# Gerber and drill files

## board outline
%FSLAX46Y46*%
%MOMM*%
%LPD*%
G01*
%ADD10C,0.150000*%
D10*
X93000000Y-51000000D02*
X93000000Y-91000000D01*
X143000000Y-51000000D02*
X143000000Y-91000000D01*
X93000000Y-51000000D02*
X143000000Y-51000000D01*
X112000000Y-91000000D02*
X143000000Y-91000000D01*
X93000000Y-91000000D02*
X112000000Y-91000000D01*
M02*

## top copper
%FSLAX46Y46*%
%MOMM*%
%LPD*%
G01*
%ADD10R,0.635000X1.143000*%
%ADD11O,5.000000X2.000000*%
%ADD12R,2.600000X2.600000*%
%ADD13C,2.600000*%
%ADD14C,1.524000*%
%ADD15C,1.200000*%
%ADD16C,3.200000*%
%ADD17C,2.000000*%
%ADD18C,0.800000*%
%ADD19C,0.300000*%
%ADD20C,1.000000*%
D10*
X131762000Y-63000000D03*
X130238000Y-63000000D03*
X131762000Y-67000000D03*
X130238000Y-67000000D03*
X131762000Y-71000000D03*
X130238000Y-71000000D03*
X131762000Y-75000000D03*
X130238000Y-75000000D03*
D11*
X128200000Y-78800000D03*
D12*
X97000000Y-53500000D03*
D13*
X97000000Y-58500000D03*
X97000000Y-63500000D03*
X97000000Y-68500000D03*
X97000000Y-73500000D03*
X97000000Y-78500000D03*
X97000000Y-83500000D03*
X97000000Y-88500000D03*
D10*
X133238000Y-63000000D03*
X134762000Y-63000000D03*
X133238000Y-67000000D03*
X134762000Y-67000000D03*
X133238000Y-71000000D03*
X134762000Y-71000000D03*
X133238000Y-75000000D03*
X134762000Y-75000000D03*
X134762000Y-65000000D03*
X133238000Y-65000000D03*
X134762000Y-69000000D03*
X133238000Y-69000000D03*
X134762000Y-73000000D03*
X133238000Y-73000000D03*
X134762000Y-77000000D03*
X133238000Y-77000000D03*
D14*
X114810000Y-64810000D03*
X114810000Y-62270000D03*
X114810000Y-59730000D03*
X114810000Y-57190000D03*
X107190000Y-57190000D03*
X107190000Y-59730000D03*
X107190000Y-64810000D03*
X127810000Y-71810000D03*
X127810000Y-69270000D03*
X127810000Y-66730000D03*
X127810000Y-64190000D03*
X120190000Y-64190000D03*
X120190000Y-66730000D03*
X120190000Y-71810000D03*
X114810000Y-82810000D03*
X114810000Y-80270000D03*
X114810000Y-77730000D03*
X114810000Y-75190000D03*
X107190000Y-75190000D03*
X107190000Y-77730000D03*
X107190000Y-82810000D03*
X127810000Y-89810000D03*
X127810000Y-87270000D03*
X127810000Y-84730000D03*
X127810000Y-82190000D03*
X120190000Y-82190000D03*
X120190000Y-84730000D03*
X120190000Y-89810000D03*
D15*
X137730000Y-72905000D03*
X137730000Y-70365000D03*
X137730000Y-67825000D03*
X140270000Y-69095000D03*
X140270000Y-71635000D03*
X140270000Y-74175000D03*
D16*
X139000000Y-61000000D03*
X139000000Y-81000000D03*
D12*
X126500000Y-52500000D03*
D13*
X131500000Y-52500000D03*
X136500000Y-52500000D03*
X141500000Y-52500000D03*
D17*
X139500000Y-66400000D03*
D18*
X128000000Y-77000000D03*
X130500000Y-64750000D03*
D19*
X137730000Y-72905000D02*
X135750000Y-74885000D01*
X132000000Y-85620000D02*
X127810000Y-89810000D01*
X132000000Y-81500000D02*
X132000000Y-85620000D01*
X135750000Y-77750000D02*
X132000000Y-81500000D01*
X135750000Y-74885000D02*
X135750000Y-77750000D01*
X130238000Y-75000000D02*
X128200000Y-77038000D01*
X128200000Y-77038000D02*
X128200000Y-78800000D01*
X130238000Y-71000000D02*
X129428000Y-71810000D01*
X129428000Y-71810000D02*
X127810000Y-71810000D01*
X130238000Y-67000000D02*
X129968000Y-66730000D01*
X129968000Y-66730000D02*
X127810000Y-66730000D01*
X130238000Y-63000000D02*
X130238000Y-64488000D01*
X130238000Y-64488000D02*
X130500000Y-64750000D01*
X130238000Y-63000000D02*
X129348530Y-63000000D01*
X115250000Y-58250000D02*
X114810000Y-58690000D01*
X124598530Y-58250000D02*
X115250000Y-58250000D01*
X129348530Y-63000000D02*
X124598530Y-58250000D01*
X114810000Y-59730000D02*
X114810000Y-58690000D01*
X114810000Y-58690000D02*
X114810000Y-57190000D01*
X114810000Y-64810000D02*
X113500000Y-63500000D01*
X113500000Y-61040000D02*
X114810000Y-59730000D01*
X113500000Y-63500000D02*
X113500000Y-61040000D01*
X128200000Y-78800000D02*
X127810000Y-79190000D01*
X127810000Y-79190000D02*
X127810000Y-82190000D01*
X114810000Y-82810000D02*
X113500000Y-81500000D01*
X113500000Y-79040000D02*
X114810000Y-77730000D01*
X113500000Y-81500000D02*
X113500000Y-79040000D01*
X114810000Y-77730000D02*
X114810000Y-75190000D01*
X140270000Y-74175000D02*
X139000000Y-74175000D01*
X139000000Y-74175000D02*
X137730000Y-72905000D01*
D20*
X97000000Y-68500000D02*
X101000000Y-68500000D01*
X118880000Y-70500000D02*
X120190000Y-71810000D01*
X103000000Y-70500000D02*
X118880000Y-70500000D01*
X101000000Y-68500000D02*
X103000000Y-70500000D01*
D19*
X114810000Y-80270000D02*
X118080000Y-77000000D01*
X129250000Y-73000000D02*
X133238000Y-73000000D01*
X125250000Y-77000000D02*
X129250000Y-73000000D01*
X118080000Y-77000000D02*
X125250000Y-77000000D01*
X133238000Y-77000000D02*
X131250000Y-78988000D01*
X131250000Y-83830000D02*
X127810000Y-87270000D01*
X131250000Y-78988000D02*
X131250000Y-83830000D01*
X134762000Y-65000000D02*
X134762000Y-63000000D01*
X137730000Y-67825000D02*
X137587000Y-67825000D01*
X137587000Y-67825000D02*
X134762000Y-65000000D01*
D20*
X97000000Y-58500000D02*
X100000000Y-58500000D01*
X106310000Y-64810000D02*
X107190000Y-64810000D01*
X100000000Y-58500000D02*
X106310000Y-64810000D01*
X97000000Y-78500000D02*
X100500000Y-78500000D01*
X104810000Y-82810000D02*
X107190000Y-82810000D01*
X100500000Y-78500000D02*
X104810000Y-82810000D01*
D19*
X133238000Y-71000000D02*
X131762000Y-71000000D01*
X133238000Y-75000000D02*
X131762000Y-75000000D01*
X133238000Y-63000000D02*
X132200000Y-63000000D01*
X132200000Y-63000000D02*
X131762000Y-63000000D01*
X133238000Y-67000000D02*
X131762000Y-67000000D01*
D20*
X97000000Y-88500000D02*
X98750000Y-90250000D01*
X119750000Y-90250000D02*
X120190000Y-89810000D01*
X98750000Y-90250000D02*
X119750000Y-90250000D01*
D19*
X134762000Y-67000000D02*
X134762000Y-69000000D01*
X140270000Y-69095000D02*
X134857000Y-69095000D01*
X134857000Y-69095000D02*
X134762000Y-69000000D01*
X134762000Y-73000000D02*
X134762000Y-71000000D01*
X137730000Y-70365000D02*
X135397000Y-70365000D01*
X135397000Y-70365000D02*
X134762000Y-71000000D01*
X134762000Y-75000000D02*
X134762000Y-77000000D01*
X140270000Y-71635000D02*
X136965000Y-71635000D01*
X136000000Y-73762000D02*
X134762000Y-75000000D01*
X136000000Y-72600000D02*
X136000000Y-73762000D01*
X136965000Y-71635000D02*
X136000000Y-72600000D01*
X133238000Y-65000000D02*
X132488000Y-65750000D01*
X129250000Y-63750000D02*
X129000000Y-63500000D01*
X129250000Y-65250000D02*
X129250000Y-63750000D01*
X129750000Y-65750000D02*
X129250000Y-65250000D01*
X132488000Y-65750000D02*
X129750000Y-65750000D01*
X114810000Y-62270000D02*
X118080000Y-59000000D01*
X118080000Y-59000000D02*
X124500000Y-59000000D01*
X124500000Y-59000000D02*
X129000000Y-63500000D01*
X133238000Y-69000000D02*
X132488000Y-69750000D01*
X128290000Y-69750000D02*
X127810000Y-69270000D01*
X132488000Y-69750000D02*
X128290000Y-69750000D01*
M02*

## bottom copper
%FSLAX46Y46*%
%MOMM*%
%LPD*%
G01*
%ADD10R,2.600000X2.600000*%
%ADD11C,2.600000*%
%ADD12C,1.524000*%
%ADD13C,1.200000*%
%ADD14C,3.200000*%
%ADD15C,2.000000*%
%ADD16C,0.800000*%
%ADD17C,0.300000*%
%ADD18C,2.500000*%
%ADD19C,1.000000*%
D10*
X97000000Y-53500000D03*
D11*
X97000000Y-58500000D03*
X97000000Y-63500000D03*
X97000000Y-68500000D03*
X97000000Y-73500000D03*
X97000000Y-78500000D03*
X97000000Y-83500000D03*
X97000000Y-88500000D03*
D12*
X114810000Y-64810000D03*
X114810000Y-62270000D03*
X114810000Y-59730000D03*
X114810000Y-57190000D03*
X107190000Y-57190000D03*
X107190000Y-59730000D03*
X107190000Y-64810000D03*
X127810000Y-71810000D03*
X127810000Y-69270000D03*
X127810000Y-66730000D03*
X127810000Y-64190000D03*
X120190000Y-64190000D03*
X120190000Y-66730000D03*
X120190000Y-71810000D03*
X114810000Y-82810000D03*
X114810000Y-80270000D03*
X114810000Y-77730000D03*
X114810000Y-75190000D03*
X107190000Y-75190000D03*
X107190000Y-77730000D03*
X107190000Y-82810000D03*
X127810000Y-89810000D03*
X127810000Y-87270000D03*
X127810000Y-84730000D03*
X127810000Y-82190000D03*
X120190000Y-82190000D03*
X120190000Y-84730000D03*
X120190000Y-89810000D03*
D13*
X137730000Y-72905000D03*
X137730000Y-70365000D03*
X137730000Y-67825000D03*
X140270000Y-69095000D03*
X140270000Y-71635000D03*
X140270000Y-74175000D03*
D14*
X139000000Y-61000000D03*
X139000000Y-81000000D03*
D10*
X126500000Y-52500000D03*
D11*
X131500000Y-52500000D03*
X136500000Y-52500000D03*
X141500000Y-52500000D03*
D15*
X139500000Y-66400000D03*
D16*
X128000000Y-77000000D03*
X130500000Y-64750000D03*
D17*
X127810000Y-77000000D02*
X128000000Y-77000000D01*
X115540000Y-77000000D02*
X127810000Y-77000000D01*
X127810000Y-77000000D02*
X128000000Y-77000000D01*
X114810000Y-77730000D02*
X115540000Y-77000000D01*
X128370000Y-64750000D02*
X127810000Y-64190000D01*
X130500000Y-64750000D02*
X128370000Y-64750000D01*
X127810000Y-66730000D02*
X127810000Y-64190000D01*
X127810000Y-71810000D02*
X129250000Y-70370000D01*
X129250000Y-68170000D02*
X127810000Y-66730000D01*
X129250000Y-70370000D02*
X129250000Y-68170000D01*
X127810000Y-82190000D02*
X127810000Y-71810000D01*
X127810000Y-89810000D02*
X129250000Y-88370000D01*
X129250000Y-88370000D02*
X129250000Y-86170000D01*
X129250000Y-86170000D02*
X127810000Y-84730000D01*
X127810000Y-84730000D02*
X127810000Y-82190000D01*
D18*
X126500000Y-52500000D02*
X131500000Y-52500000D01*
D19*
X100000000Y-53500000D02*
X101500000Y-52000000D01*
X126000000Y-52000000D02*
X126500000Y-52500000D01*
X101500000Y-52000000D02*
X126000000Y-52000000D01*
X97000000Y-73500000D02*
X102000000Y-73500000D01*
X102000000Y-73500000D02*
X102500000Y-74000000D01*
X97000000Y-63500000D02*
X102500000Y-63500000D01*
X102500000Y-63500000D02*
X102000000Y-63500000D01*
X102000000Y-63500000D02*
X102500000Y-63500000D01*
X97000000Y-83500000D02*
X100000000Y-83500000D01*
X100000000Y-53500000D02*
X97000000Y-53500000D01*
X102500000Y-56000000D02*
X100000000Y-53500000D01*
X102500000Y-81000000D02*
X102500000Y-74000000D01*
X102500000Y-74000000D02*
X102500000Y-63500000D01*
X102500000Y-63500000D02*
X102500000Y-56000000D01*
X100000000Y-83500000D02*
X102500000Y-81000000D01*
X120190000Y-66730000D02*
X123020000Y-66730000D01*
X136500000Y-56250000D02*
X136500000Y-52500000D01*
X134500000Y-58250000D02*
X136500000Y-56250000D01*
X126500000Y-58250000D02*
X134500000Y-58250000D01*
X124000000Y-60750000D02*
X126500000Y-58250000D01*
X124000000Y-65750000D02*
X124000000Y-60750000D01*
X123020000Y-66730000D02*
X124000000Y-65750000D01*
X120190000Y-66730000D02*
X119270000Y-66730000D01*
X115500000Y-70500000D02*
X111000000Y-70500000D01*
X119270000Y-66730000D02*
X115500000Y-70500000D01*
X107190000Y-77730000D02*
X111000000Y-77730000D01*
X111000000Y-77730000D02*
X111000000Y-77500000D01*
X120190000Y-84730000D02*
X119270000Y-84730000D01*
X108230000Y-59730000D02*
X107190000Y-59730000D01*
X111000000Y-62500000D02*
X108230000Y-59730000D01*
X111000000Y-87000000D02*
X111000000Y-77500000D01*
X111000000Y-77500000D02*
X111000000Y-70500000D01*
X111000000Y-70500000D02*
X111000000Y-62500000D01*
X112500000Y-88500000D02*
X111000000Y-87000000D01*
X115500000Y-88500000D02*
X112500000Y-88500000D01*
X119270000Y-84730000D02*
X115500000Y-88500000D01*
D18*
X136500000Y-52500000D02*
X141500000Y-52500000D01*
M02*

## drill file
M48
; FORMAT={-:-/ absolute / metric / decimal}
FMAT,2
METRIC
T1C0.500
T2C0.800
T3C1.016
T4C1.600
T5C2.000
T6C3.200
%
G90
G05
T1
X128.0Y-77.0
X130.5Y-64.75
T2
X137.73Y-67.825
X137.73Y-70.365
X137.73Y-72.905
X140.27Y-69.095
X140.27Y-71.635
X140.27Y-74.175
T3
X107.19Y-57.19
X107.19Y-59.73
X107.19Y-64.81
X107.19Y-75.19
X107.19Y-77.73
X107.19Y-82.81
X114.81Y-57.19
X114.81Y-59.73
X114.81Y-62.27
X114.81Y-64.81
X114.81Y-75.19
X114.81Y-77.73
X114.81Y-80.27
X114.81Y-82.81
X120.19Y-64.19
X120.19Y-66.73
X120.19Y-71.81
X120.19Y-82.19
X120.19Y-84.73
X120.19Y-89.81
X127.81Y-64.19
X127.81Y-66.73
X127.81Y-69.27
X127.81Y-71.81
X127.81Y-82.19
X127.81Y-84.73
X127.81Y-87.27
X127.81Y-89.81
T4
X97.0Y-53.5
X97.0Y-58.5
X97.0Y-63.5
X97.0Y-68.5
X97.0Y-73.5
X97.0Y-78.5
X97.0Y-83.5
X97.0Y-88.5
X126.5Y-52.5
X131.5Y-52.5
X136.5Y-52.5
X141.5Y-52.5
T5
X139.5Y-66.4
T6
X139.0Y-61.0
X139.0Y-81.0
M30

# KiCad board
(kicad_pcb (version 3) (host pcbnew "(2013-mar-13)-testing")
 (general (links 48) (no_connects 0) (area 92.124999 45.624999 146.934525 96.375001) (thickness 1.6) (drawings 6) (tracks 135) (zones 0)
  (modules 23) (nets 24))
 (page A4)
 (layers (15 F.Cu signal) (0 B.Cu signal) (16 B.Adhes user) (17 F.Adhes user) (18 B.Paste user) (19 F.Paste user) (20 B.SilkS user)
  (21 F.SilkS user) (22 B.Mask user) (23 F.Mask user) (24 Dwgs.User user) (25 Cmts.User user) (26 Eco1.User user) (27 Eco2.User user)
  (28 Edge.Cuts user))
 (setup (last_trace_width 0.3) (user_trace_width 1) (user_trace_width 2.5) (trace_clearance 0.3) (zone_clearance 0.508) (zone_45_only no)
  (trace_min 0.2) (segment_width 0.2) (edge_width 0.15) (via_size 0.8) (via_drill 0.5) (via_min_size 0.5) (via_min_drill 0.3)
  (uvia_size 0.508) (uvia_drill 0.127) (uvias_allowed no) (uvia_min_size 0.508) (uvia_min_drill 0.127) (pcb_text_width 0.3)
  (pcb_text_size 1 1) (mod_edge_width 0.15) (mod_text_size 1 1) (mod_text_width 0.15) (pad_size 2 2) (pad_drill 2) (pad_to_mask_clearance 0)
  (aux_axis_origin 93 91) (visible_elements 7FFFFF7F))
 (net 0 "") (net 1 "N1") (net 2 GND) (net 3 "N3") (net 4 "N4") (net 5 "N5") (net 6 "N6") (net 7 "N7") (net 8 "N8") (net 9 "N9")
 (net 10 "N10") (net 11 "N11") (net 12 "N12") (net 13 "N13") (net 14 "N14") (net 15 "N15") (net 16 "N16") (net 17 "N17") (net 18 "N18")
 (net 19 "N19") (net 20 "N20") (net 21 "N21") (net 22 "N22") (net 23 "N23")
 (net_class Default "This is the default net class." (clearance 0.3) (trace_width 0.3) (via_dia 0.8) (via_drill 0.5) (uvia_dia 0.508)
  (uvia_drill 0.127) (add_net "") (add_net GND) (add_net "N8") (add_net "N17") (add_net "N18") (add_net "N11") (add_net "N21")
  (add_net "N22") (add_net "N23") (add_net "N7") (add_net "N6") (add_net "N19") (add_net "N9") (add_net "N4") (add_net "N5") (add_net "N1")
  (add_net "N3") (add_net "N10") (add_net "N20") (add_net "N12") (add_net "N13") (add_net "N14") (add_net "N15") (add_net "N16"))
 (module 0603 (layer F.Cu) (at 131 63 180)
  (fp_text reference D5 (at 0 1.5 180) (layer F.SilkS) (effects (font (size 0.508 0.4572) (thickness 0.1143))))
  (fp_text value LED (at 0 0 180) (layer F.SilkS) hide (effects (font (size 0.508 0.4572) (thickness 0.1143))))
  (pad 1 smd rect (at -0.762 0 180) (size 0.635 1.143) (layers F.Cu F.Paste F.Mask) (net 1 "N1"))
  (pad 2 smd rect (at 0.762 0 180) (size 0.635 1.143) (layers F.Cu F.Paste F.Mask) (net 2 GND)))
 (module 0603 (layer F.Cu) (at 131 67 180)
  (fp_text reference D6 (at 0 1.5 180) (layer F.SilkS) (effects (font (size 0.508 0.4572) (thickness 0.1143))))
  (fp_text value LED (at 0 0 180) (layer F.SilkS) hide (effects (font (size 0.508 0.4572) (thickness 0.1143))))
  (pad 1 smd rect (at -0.762 0 180) (size 0.635 1.143) (layers F.Cu F.Paste F.Mask) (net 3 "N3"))
  (pad 2 smd rect (at 0.762 0 180) (size 0.635 1.143) (layers F.Cu F.Paste F.Mask) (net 2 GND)))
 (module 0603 (layer F.Cu) (at 131 71 180)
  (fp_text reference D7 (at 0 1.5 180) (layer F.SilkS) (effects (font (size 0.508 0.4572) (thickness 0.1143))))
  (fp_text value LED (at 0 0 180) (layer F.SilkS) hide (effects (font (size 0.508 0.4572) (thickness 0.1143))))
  (pad 1 smd rect (at -0.762 0 180) (size 0.635 1.143) (layers F.Cu F.Paste F.Mask) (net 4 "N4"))
  (pad 2 smd rect (at 0.762 0 180) (size 0.635 1.143) (layers F.Cu F.Paste F.Mask) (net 2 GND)))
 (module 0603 (layer F.Cu) (at 131 75 180)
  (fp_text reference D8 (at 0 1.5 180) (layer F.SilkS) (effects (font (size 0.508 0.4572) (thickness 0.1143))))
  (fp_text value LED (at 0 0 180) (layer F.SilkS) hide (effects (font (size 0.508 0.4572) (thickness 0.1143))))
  (pad 1 smd rect (at -0.762 0 180) (size 0.635 1.143) (layers F.Cu F.Paste F.Mask) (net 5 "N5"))
  (pad 2 smd rect (at 0.762 0 180) (size 0.635 1.143) (layers F.Cu F.Paste F.Mask) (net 2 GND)))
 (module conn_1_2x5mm (layer F.Cu) (at 128.2 78.8)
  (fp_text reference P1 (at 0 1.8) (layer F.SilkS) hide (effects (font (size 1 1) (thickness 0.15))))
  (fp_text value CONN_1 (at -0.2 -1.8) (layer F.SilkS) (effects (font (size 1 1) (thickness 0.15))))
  (pad 1 smd oval (at 0 0) (size 5 2) (layers F.Cu F.Mask) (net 2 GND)))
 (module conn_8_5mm (layer F.Cu) (at 97 71 270)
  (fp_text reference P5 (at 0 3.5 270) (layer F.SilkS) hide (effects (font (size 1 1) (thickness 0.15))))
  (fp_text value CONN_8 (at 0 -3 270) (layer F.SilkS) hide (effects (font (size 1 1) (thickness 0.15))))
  (pad 1 thru_hole rect (at -17.5 0 270) (size 2.6 2.6) (drill 1.6) (layers *.Cu *.Mask F.SilkS) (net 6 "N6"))
  (pad 2 thru_hole circle (at -12.5 0 270) (size 2.6 2.6) (drill 1.6) (layers *.Cu *.Mask F.SilkS) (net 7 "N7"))
  (pad 3 thru_hole circle (at -7.5 0 270) (size 2.6 2.6) (drill 1.6) (layers *.Cu *.Mask F.SilkS) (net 6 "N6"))
  (pad 4 thru_hole circle (at -2.5 0 270) (size 2.6 2.6) (drill 1.6) (layers *.Cu *.Mask F.SilkS) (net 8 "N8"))
  (pad 5 thru_hole circle (at 2.5 0 270) (size 2.6 2.6) (drill 1.6) (layers *.Cu *.Mask F.SilkS) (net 6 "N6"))
  (pad 6 thru_hole circle (at 7.5 0 270) (size 2.6 2.6) (drill 1.6) (layers *.Cu *.Mask F.SilkS) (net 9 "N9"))
  (pad 7 thru_hole circle (at 12.5 0 270) (size 2.6 2.6) (drill 1.6) (layers *.Cu *.Mask F.SilkS) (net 6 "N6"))
  (pad 8 thru_hole circle (at 17.5 0 270) (size 2.6 2.6) (drill 1.6) (layers *.Cu *.Mask F.SilkS) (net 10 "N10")))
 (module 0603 (layer F.Cu) (at 134 63)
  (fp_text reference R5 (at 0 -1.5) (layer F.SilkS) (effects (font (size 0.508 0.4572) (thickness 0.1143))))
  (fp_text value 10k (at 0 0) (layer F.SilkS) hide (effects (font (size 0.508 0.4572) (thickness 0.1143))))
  (pad 1 smd rect (at -0.762 0) (size 0.635 1.143) (layers F.Cu F.Paste F.Mask) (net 1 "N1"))
  (pad 2 smd rect (at 0.762 0) (size 0.635 1.143) (layers F.Cu F.Paste F.Mask) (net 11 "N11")))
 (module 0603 (layer F.Cu) (at 134 67)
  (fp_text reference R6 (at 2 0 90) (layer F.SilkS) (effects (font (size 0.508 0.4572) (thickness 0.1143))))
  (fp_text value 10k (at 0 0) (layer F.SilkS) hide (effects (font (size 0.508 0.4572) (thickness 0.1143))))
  (pad 1 smd rect (at -0.762 0) (size 0.635 1.143) (layers F.Cu F.Paste F.Mask) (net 3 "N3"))
  (pad 2 smd rect (at 0.762 0) (size 0.635 1.143) (layers F.Cu F.Paste F.Mask) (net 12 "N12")))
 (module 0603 (layer F.Cu) (at 134 71)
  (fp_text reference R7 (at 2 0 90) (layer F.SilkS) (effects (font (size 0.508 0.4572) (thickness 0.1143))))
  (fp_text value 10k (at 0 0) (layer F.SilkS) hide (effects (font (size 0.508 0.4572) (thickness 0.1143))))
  (pad 1 smd rect (at -0.762 0) (size 0.635 1.143) (layers F.Cu F.Paste F.Mask) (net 4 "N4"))
  (pad 2 smd rect (at 0.762 0) (size 0.635 1.143) (layers F.Cu F.Paste F.Mask) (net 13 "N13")))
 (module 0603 (layer F.Cu) (at 134 75)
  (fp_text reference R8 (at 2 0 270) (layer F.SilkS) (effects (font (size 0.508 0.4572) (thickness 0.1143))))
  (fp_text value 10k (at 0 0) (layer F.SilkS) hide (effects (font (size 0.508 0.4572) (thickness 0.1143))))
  (pad 1 smd rect (at -0.762 0) (size 0.635 1.143) (layers F.Cu F.Paste F.Mask) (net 5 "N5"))
  (pad 2 smd rect (at 0.762 0) (size 0.635 1.143) (layers F.Cu F.Paste F.Mask) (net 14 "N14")))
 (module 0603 (layer F.Cu) (at 134 65 180)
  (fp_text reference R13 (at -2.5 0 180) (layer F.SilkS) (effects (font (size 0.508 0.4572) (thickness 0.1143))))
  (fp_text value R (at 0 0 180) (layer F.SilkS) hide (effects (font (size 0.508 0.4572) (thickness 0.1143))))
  (pad 1 smd rect (at -0.762 0 180) (size 0.635 1.143) (layers F.Cu F.Paste F.Mask) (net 11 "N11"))
  (pad 2 smd rect (at 0.762 0 180) (size 0.635 1.143) (layers F.Cu F.Paste F.Mask) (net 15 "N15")))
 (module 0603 (layer F.Cu) (at 134 69 180)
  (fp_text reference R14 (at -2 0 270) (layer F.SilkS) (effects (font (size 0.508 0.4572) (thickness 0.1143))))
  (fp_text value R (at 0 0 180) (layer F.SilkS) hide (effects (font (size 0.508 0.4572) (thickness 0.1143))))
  (pad 1 smd rect (at -0.762 0 180) (size 0.635 1.143) (layers F.Cu F.Paste F.Mask) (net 12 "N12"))
  (pad 2 smd rect (at 0.762 0 180) (size 0.635 1.143) (layers F.Cu F.Paste F.Mask) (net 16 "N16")))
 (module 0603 (layer F.Cu) (at 134 73 180)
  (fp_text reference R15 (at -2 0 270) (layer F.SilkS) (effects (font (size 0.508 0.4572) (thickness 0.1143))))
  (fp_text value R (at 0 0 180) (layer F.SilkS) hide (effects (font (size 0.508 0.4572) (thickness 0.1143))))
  (pad 1 smd rect (at -0.762 0 180) (size 0.635 1.143) (layers F.Cu F.Paste F.Mask) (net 13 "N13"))
  (pad 2 smd rect (at 0.762 0 180) (size 0.635 1.143) (layers F.Cu F.Paste F.Mask) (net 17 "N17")))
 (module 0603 (layer F.Cu) (at 134 77 180)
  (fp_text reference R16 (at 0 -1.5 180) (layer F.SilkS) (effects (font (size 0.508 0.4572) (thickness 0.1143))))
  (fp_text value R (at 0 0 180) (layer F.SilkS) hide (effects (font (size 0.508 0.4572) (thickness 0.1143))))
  (pad 1 smd rect (at -0.762 0 180) (size 0.635 1.143) (layers F.Cu F.Paste F.Mask) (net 14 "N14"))
  (pad 2 smd rect (at 0.762 0 180) (size 0.635 1.143) (layers F.Cu F.Paste F.Mask) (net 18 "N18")))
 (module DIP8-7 (layer F.Cu) (at 111 61 180)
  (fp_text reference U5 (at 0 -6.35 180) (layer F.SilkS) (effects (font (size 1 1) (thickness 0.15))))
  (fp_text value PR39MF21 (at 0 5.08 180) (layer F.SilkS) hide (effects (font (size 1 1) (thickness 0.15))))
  (pad 1 thru_hole circle (at -3.81 -3.81 180) (size 1.524 1.524) (drill 1.016) (layers *.Cu *.Mask) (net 2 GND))
  (pad 2 thru_hole circle (at -3.81 -1.27 180) (size 1.524 1.524) (drill 1.016) (layers *.Cu *.Mask) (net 15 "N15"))
  (pad 3 thru_hole circle (at -3.81 1.27 180) (size 1.524 1.524) (drill 1.016) (layers *.Cu *.Mask) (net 2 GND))
  (pad 4 thru_hole circle (at -3.81 3.81 180) (size 1.524 1.524) (drill 1.016) (layers *.Cu *.Mask) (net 2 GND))
  (pad 5 thru_hole circle (at 3.81 3.81 180) (size 1.524 1.524) (drill 1.016) (layers *.Cu *.Mask) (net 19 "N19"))
  (pad 6 thru_hole circle (at 3.81 1.27 180) (size 1.524 1.524) (drill 1.016) (layers *.Cu *.Mask) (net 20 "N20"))
  (pad 8 thru_hole circle (at 3.81 -3.81 180) (size 1.524 1.524) (drill 1.016) (layers *.Cu *.Mask) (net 7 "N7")))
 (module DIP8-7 (layer F.Cu) (at 124 68 180)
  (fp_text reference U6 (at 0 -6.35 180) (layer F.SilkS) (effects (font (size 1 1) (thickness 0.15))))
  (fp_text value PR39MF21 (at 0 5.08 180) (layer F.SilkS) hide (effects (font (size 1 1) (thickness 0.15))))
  (pad 1 thru_hole circle (at -3.81 -3.81 180) (size 1.524 1.524) (drill 1.016) (layers *.Cu *.Mask) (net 2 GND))
  (pad 2 thru_hole circle (at -3.81 -1.27 180) (size 1.524 1.524) (drill 1.016) (layers *.Cu *.Mask) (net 16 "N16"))
  (pad 3 thru_hole circle (at -3.81 1.27 180) (size 1.524 1.524) (drill 1.016) (layers *.Cu *.Mask) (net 2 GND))
  (pad 4 thru_hole circle (at -3.81 3.81 180) (size 1.524 1.524) (drill 1.016) (layers *.Cu *.Mask) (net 2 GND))
  (pad 5 thru_hole circle (at 3.81 3.81 180) (size 1.524 1.524) (drill 1.016) (layers *.Cu *.Mask) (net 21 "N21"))
  (pad 6 thru_hole circle (at 3.81 1.27 180) (size 1.524 1.524) (drill 1.016) (layers *.Cu *.Mask) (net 20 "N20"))
  (pad 8 thru_hole circle (at 3.81 -3.81 180) (size 1.524 1.524) (drill 1.016) (layers *.Cu *.Mask) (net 8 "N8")))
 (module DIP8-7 (layer F.Cu) (at 111 79 180)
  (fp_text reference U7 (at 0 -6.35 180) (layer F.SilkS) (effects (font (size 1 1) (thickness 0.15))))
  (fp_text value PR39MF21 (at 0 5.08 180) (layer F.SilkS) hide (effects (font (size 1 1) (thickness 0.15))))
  (pad 1 thru_hole circle (at -3.81 -3.81 180) (size 1.524 1.524) (drill 1.016) (layers *.Cu *.Mask) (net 2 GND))
  (pad 2 thru_hole circle (at -3.81 -1.27 180) (size 1.524 1.524) (drill 1.016) (layers *.Cu *.Mask) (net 17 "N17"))
  (pad 3 thru_hole circle (at -3.81 1.27 180) (size 1.524 1.524) (drill 1.016) (layers *.Cu *.Mask) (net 2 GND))
  (pad 4 thru_hole circle (at -3.81 3.81 180) (size 1.524 1.524) (drill 1.016) (layers *.Cu *.Mask) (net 2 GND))
  (pad 5 thru_hole circle (at 3.81 3.81 180) (size 1.524 1.524) (drill 1.016) (layers *.Cu *.Mask) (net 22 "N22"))
  (pad 6 thru_hole circle (at 3.81 1.27 180) (size 1.524 1.524) (drill 1.016) (layers *.Cu *.Mask) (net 20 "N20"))
  (pad 8 thru_hole circle (at 3.81 -3.81 180) (size 1.524 1.524) (drill 1.016) (layers *.Cu *.Mask) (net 9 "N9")))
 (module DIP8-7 (layer F.Cu) (at 124 86 180)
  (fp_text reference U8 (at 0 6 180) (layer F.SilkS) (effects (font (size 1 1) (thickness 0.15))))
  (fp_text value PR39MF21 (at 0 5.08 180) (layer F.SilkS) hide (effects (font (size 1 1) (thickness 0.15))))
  (pad 1 thru_hole circle (at -3.81 -3.81 180) (size 1.524 1.524) (drill 1.016) (layers *.Cu *.Mask) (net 2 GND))
  (pad 2 thru_hole circle (at -3.81 -1.27 180) (size 1.524 1.524) (drill 1.016) (layers *.Cu *.Mask) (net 18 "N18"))
  (pad 3 thru_hole circle (at -3.81 1.27 180) (size 1.524 1.524) (drill 1.016) (layers *.Cu *.Mask) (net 2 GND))
  (pad 4 thru_hole circle (at -3.81 3.81 180) (size 1.524 1.524) (drill 1.016) (layers *.Cu *.Mask) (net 2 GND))
  (pad 5 thru_hole circle (at 3.81 3.81 180) (size 1.524 1.524) (drill 1.016) (layers *.Cu *.Mask) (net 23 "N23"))
  (pad 6 thru_hole circle (at 3.81 1.27 180) (size 1.524 1.524) (drill 1.016) (layers *.Cu *.Mask) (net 20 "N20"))
  (pad 8 thru_hole circle (at 3.81 -3.81 180) (size 1.524 1.524) (drill 1.016) (layers *.Cu *.Mask) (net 10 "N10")))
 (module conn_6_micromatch (layer F.Cu) (at 139 71 90)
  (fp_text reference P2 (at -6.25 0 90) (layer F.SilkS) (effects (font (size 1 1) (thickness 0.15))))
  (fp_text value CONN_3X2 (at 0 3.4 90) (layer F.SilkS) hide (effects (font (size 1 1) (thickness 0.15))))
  (pad 5 thru_hole circle (at -1.905 -1.27 90) (size 1.2 1.2) (drill 0.8) (layers *.Cu *.Mask F.SilkS) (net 2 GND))
  (pad 3 thru_hole circle (at 0.635 -1.27 90) (size 1.2 1.2) (drill 0.8) (layers *.Cu *.Mask F.SilkS) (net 13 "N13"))
  (pad 1 thru_hole circle (at 3.175 -1.27 90) (size 1.2 1.2) (drill 0.8) (layers *.Cu *.Mask F.SilkS) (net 11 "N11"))
  (pad 2 thru_hole circle (at 1.905 1.27 90) (size 1.2 1.2) (drill 0.8) (layers *.Cu *.Mask F.SilkS) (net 12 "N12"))
  (pad 4 thru_hole circle (at -0.635 1.27 90) (size 1.2 1.2) (drill 0.8) (layers *.Cu *.Mask F.SilkS) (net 14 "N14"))
  (pad 6 thru_hole circle (at -3.175 1.27 90) (size 1.2 1.2) (drill 0.8) (layers *.Cu *.Mask F.SilkS) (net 2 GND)))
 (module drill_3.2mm (layer F.Cu) (at 139 61)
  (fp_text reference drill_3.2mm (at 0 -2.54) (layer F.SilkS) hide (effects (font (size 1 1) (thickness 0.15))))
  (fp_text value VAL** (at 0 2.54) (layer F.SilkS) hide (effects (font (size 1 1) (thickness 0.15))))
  (pad "" thru_hole circle (at 0 0) (size 3.2 3.2) (drill 3.2) (layers *.Cu)))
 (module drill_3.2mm (layer F.Cu) (at 139 81)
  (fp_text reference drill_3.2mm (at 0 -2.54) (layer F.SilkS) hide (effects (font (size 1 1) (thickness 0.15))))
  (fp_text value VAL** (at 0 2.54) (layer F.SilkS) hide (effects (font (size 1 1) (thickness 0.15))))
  (pad "" thru_hole circle (at 0 0) (size 3.2 3.2) (drill 3.2) (layers *.Cu)))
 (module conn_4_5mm (layer F.Cu) (at 134 52.5)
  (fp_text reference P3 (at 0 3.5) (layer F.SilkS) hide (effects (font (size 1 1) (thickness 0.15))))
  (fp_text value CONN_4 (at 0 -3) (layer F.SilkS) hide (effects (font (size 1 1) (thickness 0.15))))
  (pad 1 thru_hole rect (at -7.5 0) (size 2.6 2.6) (drill 1.6) (layers *.Cu *.Mask F.SilkS) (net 6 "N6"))
  (pad 2 thru_hole circle (at -2.5 0) (size 2.6 2.6) (drill 1.6) (layers *.Cu *.Mask F.SilkS) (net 6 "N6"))
  (pad 3 thru_hole circle (at 2.5 0) (size 2.6 2.6) (drill 1.6) (layers *.Cu *.Mask F.SilkS) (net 20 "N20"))
  (pad 4 thru_hole circle (at 7.5 0) (size 2.6 2.6) (drill 1.6) (layers *.Cu *.Mask F.SilkS) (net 20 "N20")))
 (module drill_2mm (layer F.Cu) (at 139.5 66.4)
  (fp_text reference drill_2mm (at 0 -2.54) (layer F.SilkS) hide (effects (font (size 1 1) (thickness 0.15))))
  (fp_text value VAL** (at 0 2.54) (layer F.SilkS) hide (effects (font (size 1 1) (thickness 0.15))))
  (pad "" thru_hole circle (at 0 0) (size 2 2) (drill 2) (layers *.Cu)))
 (gr_line (start 93 51) (end 93 91) (angle 90) (layer Edge.Cuts) (width 0.15))
 (gr_line (start 143 51) (end 143 91) (angle 90) (layer Edge.Cuts) (width 0.15))
 (gr_line (start 93 51) (end 143 51) (angle 90) (layer Edge.Cuts) (width 0.15))
 (gr_line (start 112 91) (end 143 91) (angle 90) (layer Edge.Cuts) (width 0.15))
 (gr_line (start 93 91) (end 112 91) (angle 90) (layer Edge.Cuts) (width 0.15))
 (segment (start 137.73 72.905) (end 135.75 74.885) (width 0.3) (layer F.Cu) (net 2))
 (segment (start 132 85.62) (end 127.81 89.81) (width 0.3) (layer F.Cu) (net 2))
 (segment (start 132 81.5) (end 132 85.62) (width 0.3) (layer F.Cu) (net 2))
 (segment (start 135.75 77.75) (end 132 81.5) (width 0.3) (layer F.Cu) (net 2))
 (segment (start 135.75 74.885) (end 135.75 77.75) (width 0.3) (layer F.Cu) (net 2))
 (segment (start 127.81 77) (end 128 77) (width 0.3) (layer B.Cu) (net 2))
 (segment (start 115.54 77) (end 127.81 77) (width 0.3) (layer B.Cu) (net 2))
 (segment (start 127.81 77) (end 128 77) (width 0.3) (layer B.Cu) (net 2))
 (segment (start 114.81 77.73) (end 115.54 77) (width 0.3) (layer B.Cu) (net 2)) (via (at 128 77) (size 0.8) (layers F.Cu B.Cu) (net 2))
 (segment (start 130.238 75) (end 128.2 77.038) (width 0.3) (layer F.Cu) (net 2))
 (segment (start 128.2 77.038) (end 128.2 78.8) (width 0.3) (layer F.Cu) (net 2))
 (segment (start 130.238 71) (end 129.428 71.81) (width 0.3) (layer F.Cu) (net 2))
 (segment (start 129.428 71.81) (end 127.81 71.81) (width 0.3) (layer F.Cu) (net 2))
 (segment (start 130.238 67) (end 129.968 66.73) (width 0.3) (layer F.Cu) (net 2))
 (segment (start 129.968 66.73) (end 127.81 66.73) (width 0.3) (layer F.Cu) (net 2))
 (segment (start 130.238 63) (end 130.238 64.488) (width 0.3) (layer F.Cu) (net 2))
 (segment (start 128.37 64.75) (end 127.81 64.19) (width 0.3) (layer B.Cu) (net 2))
 (segment (start 130.5 64.75) (end 128.37 64.75) (width 0.3) (layer B.Cu) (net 2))
 (via (at 130.5 64.75) (size 0.8) (layers F.Cu B.Cu) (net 2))
 (segment (start 130.238 64.488) (end 130.5 64.75) (width 0.3) (layer F.Cu) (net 2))
 (segment (start 130.238 63) (end 129.34853 63) (width 0.3) (layer F.Cu) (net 2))
 (segment (start 115.25 58.25) (end 114.81 58.69) (width 0.3) (layer F.Cu) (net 2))
 (segment (start 124.59853 58.25) (end 115.25 58.25) (width 0.3) (layer F.Cu) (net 2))
 (segment (start 129.34853 63) (end 124.59853 58.25) (width 0.3) (layer F.Cu) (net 2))
 (segment (start 114.81 59.73) (end 114.81 58.69) (width 0.3) (layer F.Cu) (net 2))
 (segment (start 114.81 58.69) (end 114.81 57.19) (width 0.3) (layer F.Cu) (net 2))
 (segment (start 114.81 64.81) (end 113.5 63.5) (width 0.3) (layer F.Cu) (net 2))
 (segment (start 113.5 61.04) (end 114.81 59.73) (width 0.3) (layer F.Cu) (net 2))
 (segment (start 113.5 63.5) (end 113.5 61.04) (width 0.3) (layer F.Cu) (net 2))
 (segment (start 128.2 78.8) (end 127.81 79.19) (width 0.3) (layer F.Cu) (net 2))
 (segment (start 127.81 79.19) (end 127.81 82.19) (width 0.3) (layer F.Cu) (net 2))
 (segment (start 127.81 66.73) (end 127.81 64.19) (width 0.3) (layer B.Cu) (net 2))
 (segment (start 127.81 71.81) (end 129.25 70.37) (width 0.3) (layer B.Cu) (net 2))
 (segment (start 129.25 68.17) (end 127.81 66.73) (width 0.3) (layer B.Cu) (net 2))
 (segment (start 129.25 70.37) (end 129.25 68.17) (width 0.3) (layer B.Cu) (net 2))
 (segment (start 127.81 82.19) (end 127.81 71.81) (width 0.3) (layer B.Cu) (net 2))
 (segment (start 114.81 82.81) (end 113.5 81.5) (width 0.3) (layer F.Cu) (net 2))
 (segment (start 113.5 79.04) (end 114.81 77.73) (width 0.3) (layer F.Cu) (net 2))
 (segment (start 113.5 81.5) (end 113.5 79.04) (width 0.3) (layer F.Cu) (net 2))
 (segment (start 114.81 77.73) (end 114.81 75.19) (width 0.3) (layer F.Cu) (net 2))
 (segment (start 127.81 89.81) (end 129.25 88.37) (width 0.3) (layer B.Cu) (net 2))
 (segment (start 129.25 88.37) (end 129.25 86.17) (width 0.3) (layer B.Cu) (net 2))
 (segment (start 129.25 86.17) (end 127.81 84.73) (width 0.3) (layer B.Cu) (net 2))
 (segment (start 127.81 84.73) (end 127.81 82.19) (width 0.3) (layer B.Cu) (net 2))
 (segment (start 140.27 74.175) (end 139 74.175) (width 0.3) (layer F.Cu) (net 2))
 (segment (start 139 74.175) (end 137.73 72.905) (width 0.3) (layer F.Cu) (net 2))
 (segment (start 97 68.5) (end 101 68.5) (width 1) (layer F.Cu) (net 8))
 (segment (start 118.88 70.5) (end 120.19 71.81) (width 1) (layer F.Cu) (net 8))
 (segment (start 103 70.5) (end 118.88 70.5) (width 1) (layer F.Cu) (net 8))
 (segment (start 101 68.5) (end 103 70.5) (width 1) (layer F.Cu) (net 8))
 (segment (start 114.81 80.27) (end 118.08 77) (width 0.3) (layer F.Cu) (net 17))
 (segment (start 129.25 73) (end 133.238 73) (width 0.3) (layer F.Cu) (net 17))
 (segment (start 125.25 77) (end 129.25 73) (width 0.3) (layer F.Cu) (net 17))
 (segment (start 118.08 77) (end 125.25 77) (width 0.3) (layer F.Cu) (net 17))
 (segment (start 133.238 77) (end 131.25 78.988) (width 0.3) (layer F.Cu) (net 18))
 (segment (start 131.25 83.83) (end 127.81 87.27) (width 0.3) (layer F.Cu) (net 18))
 (segment (start 131.25 78.988) (end 131.25 83.83) (width 0.3) (layer F.Cu) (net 18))
 (segment (start 134.762 65) (end 134.762 63) (width 0.3) (layer F.Cu) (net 11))
 (segment (start 137.73 67.825) (end 137.587 67.825) (width 0.3) (layer F.Cu) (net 11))
 (segment (start 137.587 67.825) (end 134.762 65) (width 0.3) (layer F.Cu) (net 11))
 (segment (start 97 58.5) (end 100 58.5) (width 1) (layer F.Cu) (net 7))
 (segment (start 106.31 64.81) (end 107.19 64.81) (width 1) (layer F.Cu) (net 7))
 (segment (start 100 58.5) (end 106.31 64.81) (width 1) (layer F.Cu) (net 7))
 (segment (start 126.5 52.5) (end 131.5 52.5) (width 2.5) (layer B.Cu) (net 6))
 (segment (start 100 53.5) (end 101.5 52) (width 1) (layer B.Cu) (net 6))
 (segment (start 126 52) (end 126.5 52.5) (width 1) (layer B.Cu) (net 6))
 (segment (start 101.5 52) (end 126 52) (width 1) (layer B.Cu) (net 6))
 (segment (start 97 73.5) (end 102 73.5) (width 1) (layer B.Cu) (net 6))
 (segment (start 102 73.5) (end 102.5 74) (width 1) (layer B.Cu) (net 6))
 (segment (start 97 63.5) (end 102.5 63.5) (width 1) (layer B.Cu) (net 6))
 (segment (start 102.5 63.5) (end 102 63.5) (width 1) (layer B.Cu) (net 6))
 (segment (start 102 63.5) (end 102.5 63.5) (width 1) (layer B.Cu) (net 6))
 (segment (start 97 83.5) (end 100 83.5) (width 1) (layer B.Cu) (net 6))
 (segment (start 100 53.5) (end 97 53.5) (width 1) (layer B.Cu) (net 6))
 (segment (start 102.5 56) (end 100 53.5) (width 1) (layer B.Cu) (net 6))
 (segment (start 102.5 81) (end 102.5 74) (width 1) (layer B.Cu) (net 6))
 (segment (start 102.5 74) (end 102.5 63.5) (width 1) (layer B.Cu) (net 6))
 (segment (start 102.5 63.5) (end 102.5 56) (width 1) (layer B.Cu) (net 6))
 (segment (start 100 83.5) (end 102.5 81) (width 1) (layer B.Cu) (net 6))
 (segment (start 97 78.5) (end 100.5 78.5) (width 1) (layer F.Cu) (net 9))
 (segment (start 104.81 82.81) (end 107.19 82.81) (width 1) (layer F.Cu) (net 9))
 (segment (start 100.5 78.5) (end 104.81 82.81) (width 1) (layer F.Cu) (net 9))
 (segment (start 133.238 71) (end 131.762 71) (width 0.3) (layer F.Cu) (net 4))
 (segment (start 133.238 75) (end 131.762 75) (width 0.3) (layer F.Cu) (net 5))
 (segment (start 133.238 63) (end 132.2 63) (width 0.3) (layer F.Cu) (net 1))
 (segment (start 132.2 63) (end 131.762 63) (width 0.3) (layer F.Cu) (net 1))
 (segment (start 133.238 67) (end 131.762 67) (width 0.3) (layer F.Cu) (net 3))
 (segment (start 97 88.5) (end 98.75 90.25) (width 1) (layer F.Cu) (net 10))
 (segment (start 119.75 90.25) (end 120.19 89.81) (width 1) (layer F.Cu) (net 10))
 (segment (start 98.75 90.25) (end 119.75 90.25) (width 1) (layer F.Cu) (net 10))
 (segment (start 120.19 66.73) (end 123.02 66.73) (width 1) (layer B.Cu) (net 20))
 (segment (start 136.5 56.25) (end 136.5 52.5) (width 1) (layer B.Cu) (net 20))
 (segment (start 134.5 58.25) (end 136.5 56.25) (width 1) (layer B.Cu) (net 20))
 (segment (start 126.5 58.25) (end 134.5 58.25) (width 1) (layer B.Cu) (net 20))
 (segment (start 124 60.75) (end 126.5 58.25) (width 1) (layer B.Cu) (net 20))
 (segment (start 124 65.75) (end 124 60.75) (width 1) (layer B.Cu) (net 20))
 (segment (start 123.02 66.73) (end 124 65.75) (width 1) (layer B.Cu) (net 20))
 (segment (start 120.19 66.73) (end 119.27 66.73) (width 1) (layer B.Cu) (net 20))
 (segment (start 115.5 70.5) (end 111 70.5) (width 1) (layer B.Cu) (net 20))
 (segment (start 119.27 66.73) (end 115.5 70.5) (width 1) (layer B.Cu) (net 20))
 (segment (start 107.19 77.73) (end 111 77.73) (width 1) (layer B.Cu) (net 20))
 (segment (start 111 77.73) (end 111 77.5) (width 1) (layer B.Cu) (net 20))
 (segment (start 120.19 84.73) (end 119.27 84.73) (width 1) (layer B.Cu) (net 20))
 (segment (start 108.23 59.73) (end 107.19 59.73) (width 1) (layer B.Cu) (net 20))
 (segment (start 111 62.5) (end 108.23 59.73) (width 1) (layer B.Cu) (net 20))
 (segment (start 111 87) (end 111 77.5) (width 1) (layer B.Cu) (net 20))
 (segment (start 111 77.5) (end 111 70.5) (width 1) (layer B.Cu) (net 20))
 (segment (start 111 70.5) (end 111 62.5) (width 1) (layer B.Cu) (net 20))
 (segment (start 112.5 88.5) (end 111 87) (width 1) (layer B.Cu) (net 20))
 (segment (start 115.5 88.5) (end 112.5 88.5) (width 1) (layer B.Cu) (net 20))
 (segment (start 119.27 84.73) (end 115.5 88.5) (width 1) (layer B.Cu) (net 20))
 (segment (start 136.5 52.5) (end 141.5 52.5) (width 2.5) (layer B.Cu) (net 20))
 (segment (start 134.762 67) (end 134.762 69) (width 0.3) (layer F.Cu) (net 12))
 (segment (start 140.27 69.095) (end 134.857 69.095) (width 0.3) (layer F.Cu) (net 12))
 (segment (start 134.857 69.095) (end 134.762 69) (width 0.3) (layer F.Cu) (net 12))
 (segment (start 134.762 73) (end 134.762 71) (width 0.3) (layer F.Cu) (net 13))
 (segment (start 137.73 70.365) (end 135.397 70.365) (width 0.3) (layer F.Cu) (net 13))
 (segment (start 135.397 70.365) (end 134.762 71) (width 0.3) (layer F.Cu) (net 13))
 (segment (start 134.762 75) (end 134.762 77) (width 0.3) (layer F.Cu) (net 14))
 (segment (start 140.27 71.635) (end 136.965 71.635) (width 0.3) (layer F.Cu) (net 14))
 (segment (start 136 73.762) (end 134.762 75) (width 0.3) (layer F.Cu) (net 14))
 (segment (start 136 72.6) (end 136 73.762) (width 0.3) (layer F.Cu) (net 14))
 (segment (start 136.965 71.635) (end 136 72.6) (width 0.3) (layer F.Cu) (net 14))
 (segment (start 133.238 65) (end 132.488 65.75) (width 0.3) (layer F.Cu) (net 15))
 (segment (start 129.25 63.75) (end 129 63.5) (width 0.3) (layer F.Cu) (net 15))
 (segment (start 129.25 65.25) (end 129.25 63.75) (width 0.3) (layer F.Cu) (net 15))
 (segment (start 129.75 65.75) (end 129.25 65.25) (width 0.3) (layer F.Cu) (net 15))
 (segment (start 132.488 65.75) (end 129.75 65.75) (width 0.3) (layer F.Cu) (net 15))
 (segment (start 114.81 62.27) (end 118.08 59) (width 0.3) (layer F.Cu) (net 15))
 (segment (start 118.08 59) (end 124.5 59) (width 0.3) (layer F.Cu) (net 15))
 (segment (start 124.5 59) (end 129 63.5) (width 0.3) (layer F.Cu) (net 15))
 (segment (start 133.238 69) (end 132.488 69.75) (width 0.3) (layer F.Cu) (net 16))
 (segment (start 128.29 69.75) (end 127.81 69.27) (width 0.3) (layer F.Cu) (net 16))
 (segment (start 132.488 69.75) (end 128.29 69.75) (width 0.3) (layer F.Cu) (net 16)))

